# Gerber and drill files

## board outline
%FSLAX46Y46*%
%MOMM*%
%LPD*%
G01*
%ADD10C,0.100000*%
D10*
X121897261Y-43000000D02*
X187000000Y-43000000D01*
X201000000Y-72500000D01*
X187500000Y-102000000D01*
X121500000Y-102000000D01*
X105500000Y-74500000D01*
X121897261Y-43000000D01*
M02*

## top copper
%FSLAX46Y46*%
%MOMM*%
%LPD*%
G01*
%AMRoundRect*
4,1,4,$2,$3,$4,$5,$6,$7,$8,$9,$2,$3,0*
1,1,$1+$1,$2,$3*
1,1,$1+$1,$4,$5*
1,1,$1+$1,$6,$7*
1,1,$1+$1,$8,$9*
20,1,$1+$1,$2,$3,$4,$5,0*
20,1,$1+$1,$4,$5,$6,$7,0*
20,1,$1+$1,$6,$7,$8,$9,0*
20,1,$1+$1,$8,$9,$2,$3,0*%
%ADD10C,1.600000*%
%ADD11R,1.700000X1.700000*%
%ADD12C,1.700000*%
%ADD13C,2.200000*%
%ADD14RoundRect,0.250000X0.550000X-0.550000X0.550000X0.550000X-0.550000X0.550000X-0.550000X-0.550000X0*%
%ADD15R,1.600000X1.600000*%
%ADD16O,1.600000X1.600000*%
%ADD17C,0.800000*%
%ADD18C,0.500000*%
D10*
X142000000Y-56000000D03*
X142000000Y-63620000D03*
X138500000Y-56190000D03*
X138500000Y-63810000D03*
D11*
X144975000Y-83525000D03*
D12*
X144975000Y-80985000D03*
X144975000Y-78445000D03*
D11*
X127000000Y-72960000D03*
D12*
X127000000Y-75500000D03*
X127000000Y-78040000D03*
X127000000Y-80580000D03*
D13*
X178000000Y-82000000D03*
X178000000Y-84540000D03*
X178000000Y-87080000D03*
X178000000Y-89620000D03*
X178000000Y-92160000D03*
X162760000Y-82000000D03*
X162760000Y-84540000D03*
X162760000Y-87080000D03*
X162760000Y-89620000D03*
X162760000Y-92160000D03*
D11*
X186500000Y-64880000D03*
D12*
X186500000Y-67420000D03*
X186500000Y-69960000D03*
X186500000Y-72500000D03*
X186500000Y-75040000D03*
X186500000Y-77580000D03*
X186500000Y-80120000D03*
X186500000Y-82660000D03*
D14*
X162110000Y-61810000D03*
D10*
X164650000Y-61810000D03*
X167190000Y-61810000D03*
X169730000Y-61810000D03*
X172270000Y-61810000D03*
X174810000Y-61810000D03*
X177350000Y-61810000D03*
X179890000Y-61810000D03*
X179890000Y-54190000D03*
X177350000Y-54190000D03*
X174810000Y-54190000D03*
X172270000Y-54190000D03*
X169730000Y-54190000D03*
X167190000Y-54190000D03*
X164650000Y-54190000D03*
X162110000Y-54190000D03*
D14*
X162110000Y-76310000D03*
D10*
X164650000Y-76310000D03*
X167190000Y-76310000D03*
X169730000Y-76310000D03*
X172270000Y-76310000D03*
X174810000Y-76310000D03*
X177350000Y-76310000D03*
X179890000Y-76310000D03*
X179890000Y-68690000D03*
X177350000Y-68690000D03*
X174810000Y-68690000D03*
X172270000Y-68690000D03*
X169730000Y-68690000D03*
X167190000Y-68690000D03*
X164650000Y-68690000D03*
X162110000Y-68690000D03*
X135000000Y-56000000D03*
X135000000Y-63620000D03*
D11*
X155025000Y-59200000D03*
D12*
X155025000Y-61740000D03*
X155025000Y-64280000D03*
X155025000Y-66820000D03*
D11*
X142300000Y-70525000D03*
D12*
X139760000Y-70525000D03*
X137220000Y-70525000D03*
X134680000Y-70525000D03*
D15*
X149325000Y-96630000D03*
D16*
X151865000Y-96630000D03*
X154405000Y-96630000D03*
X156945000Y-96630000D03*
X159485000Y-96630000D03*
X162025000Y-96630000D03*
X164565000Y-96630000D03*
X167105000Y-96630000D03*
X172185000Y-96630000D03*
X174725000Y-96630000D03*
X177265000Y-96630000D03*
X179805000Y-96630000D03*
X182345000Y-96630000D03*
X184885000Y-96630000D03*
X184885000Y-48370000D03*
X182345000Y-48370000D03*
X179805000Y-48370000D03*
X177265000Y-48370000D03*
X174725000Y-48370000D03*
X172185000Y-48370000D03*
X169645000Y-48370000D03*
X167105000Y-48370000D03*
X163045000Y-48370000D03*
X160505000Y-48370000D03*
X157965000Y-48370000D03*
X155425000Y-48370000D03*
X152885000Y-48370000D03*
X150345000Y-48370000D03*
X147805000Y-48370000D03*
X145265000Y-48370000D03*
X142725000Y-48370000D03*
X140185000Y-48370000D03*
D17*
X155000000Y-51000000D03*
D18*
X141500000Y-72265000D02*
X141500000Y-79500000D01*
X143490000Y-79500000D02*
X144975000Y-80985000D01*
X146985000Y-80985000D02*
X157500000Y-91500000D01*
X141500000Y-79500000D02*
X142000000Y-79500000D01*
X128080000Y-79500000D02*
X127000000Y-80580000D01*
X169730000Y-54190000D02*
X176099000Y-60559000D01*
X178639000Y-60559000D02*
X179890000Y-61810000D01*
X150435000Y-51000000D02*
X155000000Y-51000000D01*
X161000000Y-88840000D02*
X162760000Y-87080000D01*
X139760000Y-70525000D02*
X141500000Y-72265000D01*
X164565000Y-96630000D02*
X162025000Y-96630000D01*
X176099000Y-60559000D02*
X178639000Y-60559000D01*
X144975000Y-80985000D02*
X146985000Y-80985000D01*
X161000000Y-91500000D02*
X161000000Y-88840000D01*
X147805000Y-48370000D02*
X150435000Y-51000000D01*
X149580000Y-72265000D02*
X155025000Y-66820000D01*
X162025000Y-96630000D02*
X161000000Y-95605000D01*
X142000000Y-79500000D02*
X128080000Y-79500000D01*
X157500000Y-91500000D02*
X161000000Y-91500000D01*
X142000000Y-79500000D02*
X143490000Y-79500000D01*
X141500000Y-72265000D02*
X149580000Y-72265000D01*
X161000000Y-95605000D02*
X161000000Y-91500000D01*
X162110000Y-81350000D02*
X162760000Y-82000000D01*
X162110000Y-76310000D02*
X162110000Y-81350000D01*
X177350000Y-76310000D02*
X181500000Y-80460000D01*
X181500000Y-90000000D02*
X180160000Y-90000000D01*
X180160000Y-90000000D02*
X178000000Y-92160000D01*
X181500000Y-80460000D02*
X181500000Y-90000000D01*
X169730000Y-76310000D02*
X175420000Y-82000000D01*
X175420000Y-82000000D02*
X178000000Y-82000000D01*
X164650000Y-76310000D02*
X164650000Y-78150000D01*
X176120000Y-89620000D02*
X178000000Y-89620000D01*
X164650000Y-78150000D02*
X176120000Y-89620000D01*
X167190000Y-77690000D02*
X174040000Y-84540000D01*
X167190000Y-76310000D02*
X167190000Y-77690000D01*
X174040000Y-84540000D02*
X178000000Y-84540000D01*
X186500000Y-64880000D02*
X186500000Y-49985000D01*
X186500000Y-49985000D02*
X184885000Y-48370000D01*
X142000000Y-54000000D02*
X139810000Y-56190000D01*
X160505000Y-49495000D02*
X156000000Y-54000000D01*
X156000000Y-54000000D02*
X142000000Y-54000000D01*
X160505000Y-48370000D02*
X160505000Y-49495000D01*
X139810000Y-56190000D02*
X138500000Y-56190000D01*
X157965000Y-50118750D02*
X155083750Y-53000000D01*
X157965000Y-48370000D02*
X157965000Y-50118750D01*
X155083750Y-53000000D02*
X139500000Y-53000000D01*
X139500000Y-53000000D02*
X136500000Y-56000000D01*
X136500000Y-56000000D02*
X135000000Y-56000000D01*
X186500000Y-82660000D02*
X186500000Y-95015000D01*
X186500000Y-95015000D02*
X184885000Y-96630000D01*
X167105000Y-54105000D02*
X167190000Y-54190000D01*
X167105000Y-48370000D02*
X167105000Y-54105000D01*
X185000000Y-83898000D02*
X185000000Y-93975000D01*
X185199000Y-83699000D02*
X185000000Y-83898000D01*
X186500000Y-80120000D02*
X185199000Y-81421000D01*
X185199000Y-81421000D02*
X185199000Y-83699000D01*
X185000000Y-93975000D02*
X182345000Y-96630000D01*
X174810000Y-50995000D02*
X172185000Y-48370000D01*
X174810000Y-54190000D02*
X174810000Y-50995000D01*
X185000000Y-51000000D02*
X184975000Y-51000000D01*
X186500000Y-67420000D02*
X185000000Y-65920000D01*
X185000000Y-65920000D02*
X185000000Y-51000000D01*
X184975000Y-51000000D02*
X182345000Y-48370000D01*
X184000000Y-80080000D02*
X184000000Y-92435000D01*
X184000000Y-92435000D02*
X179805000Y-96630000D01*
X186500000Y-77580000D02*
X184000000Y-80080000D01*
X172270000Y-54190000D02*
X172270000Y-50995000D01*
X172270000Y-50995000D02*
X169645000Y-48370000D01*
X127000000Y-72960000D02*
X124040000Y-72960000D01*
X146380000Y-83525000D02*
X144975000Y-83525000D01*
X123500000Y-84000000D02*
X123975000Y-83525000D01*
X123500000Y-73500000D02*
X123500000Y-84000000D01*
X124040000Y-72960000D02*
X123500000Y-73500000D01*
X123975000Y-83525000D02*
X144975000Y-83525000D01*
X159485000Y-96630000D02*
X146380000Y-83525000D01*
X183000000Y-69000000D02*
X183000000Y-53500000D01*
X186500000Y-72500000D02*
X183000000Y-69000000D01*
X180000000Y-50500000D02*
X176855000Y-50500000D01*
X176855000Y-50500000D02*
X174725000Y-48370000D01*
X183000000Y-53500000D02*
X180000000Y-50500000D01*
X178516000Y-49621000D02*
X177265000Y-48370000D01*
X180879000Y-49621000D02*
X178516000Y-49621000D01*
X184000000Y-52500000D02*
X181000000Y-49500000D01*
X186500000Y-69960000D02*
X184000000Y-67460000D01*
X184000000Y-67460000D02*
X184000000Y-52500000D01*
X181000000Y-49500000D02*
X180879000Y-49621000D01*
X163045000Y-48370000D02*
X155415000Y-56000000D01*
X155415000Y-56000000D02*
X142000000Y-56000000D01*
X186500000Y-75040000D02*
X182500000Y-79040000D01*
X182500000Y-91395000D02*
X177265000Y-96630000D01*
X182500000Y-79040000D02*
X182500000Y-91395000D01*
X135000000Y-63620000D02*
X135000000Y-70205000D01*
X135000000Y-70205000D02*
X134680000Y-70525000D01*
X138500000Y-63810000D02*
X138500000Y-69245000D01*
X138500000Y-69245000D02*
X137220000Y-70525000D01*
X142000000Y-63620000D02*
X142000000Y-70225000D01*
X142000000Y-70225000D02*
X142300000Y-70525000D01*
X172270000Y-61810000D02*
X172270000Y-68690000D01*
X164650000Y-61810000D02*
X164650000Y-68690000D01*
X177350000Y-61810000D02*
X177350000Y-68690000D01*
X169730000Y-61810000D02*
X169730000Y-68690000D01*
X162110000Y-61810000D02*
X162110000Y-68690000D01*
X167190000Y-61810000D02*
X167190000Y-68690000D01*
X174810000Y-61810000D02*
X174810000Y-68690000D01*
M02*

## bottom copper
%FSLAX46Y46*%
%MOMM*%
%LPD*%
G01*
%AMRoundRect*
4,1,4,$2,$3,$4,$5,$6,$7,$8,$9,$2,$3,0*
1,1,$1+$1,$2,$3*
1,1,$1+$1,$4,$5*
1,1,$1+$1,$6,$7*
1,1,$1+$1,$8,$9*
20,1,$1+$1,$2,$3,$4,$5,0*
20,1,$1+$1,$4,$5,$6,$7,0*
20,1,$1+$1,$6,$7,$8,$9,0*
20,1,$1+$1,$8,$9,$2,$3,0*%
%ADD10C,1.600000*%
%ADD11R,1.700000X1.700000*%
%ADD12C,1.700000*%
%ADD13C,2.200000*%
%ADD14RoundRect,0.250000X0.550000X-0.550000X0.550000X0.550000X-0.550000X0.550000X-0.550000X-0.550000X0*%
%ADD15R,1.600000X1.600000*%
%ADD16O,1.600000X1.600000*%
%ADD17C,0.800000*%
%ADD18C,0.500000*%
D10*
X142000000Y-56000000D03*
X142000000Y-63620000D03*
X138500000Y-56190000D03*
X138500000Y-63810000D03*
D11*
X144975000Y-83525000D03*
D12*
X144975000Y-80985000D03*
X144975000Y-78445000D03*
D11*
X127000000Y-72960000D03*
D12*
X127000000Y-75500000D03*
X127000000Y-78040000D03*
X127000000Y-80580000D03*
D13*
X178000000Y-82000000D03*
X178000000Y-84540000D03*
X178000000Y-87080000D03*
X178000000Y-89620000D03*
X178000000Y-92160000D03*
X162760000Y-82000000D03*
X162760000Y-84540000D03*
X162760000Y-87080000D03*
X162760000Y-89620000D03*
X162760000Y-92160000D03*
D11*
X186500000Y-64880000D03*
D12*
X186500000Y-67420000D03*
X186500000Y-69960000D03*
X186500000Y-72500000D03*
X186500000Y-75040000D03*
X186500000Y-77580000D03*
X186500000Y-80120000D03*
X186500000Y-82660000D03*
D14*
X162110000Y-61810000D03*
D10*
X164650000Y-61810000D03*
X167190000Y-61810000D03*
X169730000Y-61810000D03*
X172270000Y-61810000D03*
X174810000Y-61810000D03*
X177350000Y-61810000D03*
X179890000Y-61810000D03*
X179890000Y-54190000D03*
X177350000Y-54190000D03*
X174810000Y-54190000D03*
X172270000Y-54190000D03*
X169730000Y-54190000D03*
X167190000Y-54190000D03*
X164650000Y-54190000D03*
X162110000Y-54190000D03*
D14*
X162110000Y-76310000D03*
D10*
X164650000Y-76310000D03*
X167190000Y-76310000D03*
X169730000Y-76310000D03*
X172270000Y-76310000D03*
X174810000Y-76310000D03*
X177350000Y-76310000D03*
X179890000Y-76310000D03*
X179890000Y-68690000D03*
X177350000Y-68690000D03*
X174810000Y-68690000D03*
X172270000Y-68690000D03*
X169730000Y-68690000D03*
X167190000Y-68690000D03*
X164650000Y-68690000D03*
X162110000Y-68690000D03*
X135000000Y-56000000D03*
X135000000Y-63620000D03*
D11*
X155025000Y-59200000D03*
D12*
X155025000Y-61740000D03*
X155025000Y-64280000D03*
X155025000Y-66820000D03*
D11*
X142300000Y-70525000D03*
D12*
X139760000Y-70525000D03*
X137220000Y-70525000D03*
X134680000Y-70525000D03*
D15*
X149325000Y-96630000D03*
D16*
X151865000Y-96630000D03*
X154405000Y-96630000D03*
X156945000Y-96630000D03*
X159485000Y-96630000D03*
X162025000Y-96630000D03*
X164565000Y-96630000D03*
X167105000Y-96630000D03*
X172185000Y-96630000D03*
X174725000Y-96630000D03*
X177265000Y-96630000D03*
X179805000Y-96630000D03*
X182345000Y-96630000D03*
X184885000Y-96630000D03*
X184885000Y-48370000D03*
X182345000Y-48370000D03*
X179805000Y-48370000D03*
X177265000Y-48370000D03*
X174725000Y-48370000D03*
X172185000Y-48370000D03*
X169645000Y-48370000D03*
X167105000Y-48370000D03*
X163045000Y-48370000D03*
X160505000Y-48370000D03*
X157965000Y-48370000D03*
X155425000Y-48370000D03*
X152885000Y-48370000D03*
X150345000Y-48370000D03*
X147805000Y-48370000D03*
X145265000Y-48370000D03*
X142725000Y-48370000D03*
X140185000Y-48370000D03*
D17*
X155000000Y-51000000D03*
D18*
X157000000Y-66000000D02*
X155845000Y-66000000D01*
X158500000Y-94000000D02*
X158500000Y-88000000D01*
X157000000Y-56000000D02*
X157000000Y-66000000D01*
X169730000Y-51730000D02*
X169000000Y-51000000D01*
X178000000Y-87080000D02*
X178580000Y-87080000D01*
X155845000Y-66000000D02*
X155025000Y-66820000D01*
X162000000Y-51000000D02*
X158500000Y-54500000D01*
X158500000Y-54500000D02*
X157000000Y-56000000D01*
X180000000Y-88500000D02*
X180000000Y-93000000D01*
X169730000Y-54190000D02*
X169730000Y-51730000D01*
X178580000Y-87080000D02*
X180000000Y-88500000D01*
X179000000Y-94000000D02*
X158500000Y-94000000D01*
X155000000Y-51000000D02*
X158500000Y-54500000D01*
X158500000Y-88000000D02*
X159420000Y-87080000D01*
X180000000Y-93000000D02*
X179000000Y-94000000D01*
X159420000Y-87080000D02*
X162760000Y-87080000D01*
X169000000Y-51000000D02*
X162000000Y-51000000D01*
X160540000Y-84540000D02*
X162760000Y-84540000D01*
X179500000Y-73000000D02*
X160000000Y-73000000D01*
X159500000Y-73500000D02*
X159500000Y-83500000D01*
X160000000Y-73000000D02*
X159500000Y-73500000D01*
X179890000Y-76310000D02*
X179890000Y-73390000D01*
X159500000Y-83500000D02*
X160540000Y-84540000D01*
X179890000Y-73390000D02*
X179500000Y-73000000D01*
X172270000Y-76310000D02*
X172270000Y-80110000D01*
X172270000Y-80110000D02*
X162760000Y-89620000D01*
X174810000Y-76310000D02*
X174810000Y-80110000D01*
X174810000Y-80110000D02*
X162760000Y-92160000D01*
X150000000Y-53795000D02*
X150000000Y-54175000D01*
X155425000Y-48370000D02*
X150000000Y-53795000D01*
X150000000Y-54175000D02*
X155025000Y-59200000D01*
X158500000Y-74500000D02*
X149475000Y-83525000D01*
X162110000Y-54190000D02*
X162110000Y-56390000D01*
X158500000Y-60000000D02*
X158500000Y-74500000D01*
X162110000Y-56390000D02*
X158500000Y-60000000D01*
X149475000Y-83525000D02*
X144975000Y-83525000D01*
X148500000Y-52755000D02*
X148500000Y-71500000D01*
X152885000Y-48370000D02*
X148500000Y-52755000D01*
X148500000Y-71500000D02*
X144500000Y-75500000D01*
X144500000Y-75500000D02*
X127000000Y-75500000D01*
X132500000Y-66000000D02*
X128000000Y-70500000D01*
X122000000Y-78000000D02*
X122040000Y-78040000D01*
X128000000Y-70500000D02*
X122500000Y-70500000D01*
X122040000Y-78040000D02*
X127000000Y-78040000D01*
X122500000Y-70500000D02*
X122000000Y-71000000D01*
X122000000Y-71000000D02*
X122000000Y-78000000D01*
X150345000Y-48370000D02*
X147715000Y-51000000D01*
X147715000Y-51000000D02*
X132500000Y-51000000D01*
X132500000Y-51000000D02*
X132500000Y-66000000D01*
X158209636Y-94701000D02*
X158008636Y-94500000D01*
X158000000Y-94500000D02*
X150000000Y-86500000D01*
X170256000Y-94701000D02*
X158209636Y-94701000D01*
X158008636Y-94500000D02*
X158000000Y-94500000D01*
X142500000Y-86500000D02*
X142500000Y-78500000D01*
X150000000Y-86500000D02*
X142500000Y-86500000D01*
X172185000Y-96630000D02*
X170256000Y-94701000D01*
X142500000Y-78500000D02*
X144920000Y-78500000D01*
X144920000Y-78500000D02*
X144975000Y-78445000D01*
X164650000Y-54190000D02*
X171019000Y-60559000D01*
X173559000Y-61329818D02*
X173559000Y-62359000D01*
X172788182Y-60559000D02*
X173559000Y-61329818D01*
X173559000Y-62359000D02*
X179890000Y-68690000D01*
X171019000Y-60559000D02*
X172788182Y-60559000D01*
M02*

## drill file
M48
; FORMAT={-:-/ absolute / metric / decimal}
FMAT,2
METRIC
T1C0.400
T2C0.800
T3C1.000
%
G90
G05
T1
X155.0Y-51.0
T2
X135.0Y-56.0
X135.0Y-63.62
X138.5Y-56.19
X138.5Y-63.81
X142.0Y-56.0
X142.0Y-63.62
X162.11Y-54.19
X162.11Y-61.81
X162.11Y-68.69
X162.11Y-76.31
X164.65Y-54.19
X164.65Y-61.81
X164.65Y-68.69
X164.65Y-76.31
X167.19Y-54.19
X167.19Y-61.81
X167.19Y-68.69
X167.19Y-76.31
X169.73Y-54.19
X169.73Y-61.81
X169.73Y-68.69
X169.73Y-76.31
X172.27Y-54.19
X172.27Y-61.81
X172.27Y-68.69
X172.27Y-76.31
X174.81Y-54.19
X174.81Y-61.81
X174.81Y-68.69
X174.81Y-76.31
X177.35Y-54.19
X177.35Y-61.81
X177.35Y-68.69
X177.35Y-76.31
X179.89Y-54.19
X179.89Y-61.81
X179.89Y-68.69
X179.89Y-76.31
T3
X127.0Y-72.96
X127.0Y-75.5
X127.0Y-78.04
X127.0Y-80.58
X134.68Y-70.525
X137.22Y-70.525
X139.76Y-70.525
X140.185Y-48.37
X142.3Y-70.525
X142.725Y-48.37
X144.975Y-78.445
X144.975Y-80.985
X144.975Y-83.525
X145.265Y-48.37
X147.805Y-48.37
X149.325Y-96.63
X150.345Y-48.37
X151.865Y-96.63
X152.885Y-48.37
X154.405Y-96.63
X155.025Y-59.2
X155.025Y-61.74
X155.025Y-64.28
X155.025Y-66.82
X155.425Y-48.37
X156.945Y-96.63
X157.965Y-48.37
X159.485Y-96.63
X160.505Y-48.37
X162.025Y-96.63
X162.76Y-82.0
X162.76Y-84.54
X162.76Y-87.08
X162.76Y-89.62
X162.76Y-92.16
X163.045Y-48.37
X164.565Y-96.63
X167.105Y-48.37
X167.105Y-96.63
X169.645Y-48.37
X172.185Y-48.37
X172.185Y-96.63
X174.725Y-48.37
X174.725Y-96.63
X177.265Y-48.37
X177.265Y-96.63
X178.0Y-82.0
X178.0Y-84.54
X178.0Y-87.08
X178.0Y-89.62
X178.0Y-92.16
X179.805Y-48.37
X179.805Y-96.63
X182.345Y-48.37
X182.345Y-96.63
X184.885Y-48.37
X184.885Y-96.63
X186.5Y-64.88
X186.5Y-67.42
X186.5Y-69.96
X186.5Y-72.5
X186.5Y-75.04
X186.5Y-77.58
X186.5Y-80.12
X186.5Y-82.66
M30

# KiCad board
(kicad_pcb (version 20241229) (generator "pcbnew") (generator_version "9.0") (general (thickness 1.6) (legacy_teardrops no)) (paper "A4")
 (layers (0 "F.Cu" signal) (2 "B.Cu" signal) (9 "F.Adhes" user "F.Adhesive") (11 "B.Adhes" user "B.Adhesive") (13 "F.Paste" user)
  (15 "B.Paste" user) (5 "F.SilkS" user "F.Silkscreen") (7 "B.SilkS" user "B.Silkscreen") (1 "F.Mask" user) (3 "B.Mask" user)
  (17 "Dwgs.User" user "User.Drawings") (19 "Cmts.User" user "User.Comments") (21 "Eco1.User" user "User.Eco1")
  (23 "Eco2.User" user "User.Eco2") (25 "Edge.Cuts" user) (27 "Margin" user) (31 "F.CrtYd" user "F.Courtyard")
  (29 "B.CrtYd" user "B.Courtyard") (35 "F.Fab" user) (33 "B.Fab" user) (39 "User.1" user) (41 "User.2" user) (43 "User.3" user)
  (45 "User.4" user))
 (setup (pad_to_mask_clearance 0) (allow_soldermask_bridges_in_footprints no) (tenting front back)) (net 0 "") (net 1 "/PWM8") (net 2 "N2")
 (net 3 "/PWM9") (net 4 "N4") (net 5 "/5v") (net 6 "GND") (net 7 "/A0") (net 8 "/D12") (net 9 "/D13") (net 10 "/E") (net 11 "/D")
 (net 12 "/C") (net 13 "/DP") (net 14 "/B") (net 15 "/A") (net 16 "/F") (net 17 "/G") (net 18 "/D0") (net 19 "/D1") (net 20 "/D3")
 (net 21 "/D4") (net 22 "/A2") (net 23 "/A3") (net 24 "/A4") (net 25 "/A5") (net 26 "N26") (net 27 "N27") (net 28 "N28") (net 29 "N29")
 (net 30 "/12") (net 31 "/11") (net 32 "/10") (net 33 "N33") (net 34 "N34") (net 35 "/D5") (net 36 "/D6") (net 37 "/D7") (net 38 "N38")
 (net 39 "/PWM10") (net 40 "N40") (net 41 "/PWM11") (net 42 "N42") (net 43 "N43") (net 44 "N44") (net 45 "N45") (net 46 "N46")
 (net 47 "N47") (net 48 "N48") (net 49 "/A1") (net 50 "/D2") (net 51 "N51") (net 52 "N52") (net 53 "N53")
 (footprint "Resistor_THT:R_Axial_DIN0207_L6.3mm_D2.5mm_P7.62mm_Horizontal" (layer "F.Cu") (at 142 56 -90)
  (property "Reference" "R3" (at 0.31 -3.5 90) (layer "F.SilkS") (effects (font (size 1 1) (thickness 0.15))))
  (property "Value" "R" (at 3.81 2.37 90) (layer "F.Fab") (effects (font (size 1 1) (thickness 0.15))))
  (pad "1" thru_hole circle (at 0 0 270) (size 1.6 1.6) (drill 0.8) (layers "*.Cu" "*.Mask") (remove_unused_layers no) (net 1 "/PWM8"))
  (pad "2" thru_hole circle (at 7.62 0 270) (size 1.6 1.6) (drill 0.8) (layers "*.Cu" "*.Mask") (remove_unused_layers no) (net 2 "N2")))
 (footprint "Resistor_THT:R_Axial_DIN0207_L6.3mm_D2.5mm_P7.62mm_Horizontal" (layer "F.Cu") (at 138.5 56.19 -90)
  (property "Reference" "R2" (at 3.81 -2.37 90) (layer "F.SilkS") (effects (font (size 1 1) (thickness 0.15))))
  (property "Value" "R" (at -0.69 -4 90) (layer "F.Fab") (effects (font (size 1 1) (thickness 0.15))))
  (pad "1" thru_hole circle (at 0 0 270) (size 1.6 1.6) (drill 0.8) (layers "*.Cu" "*.Mask") (remove_unused_layers no) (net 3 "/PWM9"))
  (pad "2" thru_hole circle (at 7.62 0 270) (size 1.6 1.6) (drill 0.8) (layers "*.Cu" "*.Mask") (remove_unused_layers no) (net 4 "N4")))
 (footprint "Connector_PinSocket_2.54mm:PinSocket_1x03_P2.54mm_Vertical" (layer "F.Cu") (at 144.975 83.525 180)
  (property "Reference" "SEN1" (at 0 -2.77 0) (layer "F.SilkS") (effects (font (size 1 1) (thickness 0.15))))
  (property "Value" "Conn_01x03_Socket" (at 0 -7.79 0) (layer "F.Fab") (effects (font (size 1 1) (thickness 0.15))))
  (pad "1" thru_hole rect (at 0 0 180) (size 1.7 1.7) (drill 1) (layers "*.Cu" "*.Mask") (remove_unused_layers no) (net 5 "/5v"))
  (pad "2" thru_hole circle (at 0 2.54 180) (size 1.7 1.7) (drill 1) (layers "*.Cu" "*.Mask") (remove_unused_layers no) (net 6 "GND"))
  (pad "3" thru_hole circle (at 0 5.08 180) (size 1.7 1.7) (drill 1) (layers "*.Cu" "*.Mask") (remove_unused_layers no) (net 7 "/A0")))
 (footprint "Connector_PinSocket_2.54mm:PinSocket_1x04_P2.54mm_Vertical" (layer "F.Cu") (at 127 72.96)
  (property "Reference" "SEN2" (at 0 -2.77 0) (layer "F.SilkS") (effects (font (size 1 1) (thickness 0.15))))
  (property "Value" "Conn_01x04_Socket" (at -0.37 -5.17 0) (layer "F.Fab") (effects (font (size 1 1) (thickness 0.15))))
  (pad "1" thru_hole rect (at 0 0) (size 1.7 1.7) (drill 1) (layers "*.Cu" "*.Mask") (remove_unused_layers no) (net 5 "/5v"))
  (pad "2" thru_hole circle (at 0 2.54) (size 1.7 1.7) (drill 1) (layers "*.Cu" "*.Mask") (remove_unused_layers no) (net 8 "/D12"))
  (pad "3" thru_hole circle (at 0 5.08) (size 1.7 1.7) (drill 1) (layers "*.Cu" "*.Mask") (remove_unused_layers no) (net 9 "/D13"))
  (pad "4" thru_hole circle (at 0 7.62) (size 1.7 1.7) (drill 1) (layers "*.Cu" "*.Mask") (remove_unused_layers no) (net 6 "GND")))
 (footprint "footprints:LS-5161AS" (layer "F.Cu") (at 178 82 -90)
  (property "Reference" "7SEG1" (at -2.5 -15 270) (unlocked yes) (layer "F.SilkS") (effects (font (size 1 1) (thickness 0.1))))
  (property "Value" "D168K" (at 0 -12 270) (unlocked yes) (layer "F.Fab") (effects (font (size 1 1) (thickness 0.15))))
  (pad "1" thru_hole circle (at 0 0 270) (size 2.2 2.2) (drill 1) (layers "*.Cu" "*.Mask") (remove_unused_layers no) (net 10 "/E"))
  (pad "2" thru_hole circle (at 2.54 0 270) (size 2.2 2.2) (drill 1) (layers "*.Cu" "*.Mask") (remove_unused_layers no) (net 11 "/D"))
  (pad "3" thru_hole circle (at 5.08 0 270) (size 2.2 2.2) (drill 1) (layers "*.Cu" "*.Mask") (remove_unused_layers no) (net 6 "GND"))
  (pad "4" thru_hole circle (at 7.62 0 270) (size 2.2 2.2) (drill 1) (layers "*.Cu" "*.Mask") (remove_unused_layers no) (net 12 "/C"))
  (pad "5" thru_hole circle (at 10.16 0 270) (size 2.2 2.2) (drill 1) (layers "*.Cu" "*.Mask") (remove_unused_layers no) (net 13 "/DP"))
  (pad "6" thru_hole circle (at 0 15.24 270) (size 2.2 2.2) (drill 1) (layers "*.Cu" "*.Mask") (remove_unused_layers no) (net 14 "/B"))
  (pad "7" thru_hole circle (at 2.54 15.24 270) (size 2.2 2.2) (drill 1) (layers "*.Cu" "*.Mask") (remove_unused_layers no) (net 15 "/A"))
  (pad "8" thru_hole circle (at 5.08 15.24 270) (size 2.2 2.2) (drill 1) (layers "*.Cu" "*.Mask") (remove_unused_layers no) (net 6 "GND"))
  (pad "9" thru_hole circle (at 7.62 15.24 270) (size 2.2 2.2) (drill 1) (layers "*.Cu" "*.Mask") (remove_unused_layers no) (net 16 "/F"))
  (pad "10" thru_hole circle (at 10.16 15.24 270) (size 2.2 2.2) (drill 1) (layers "*.Cu" "*.Mask") (remove_unused_layers no) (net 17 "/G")))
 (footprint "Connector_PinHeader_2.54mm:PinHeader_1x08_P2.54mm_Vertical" (layer "F.Cu") (at 186.5 64.88)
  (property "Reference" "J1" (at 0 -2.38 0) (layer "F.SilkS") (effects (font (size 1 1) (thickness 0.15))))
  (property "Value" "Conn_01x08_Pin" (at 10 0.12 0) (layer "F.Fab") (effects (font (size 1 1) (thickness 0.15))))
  (pad "1" thru_hole rect (at 0 0) (size 1.7 1.7) (drill 1) (layers "*.Cu" "*.Mask") (remove_unused_layers no) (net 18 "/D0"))
  (pad "2" thru_hole circle (at 0 2.54) (size 1.7 1.7) (drill 1) (layers "*.Cu" "*.Mask") (remove_unused_layers no) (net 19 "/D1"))
  (pad "3" thru_hole circle (at 0 5.08) (size 1.7 1.7) (drill 1) (layers "*.Cu" "*.Mask") (remove_unused_layers no) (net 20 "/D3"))
  (pad "4" thru_hole circle (at 0 7.62) (size 1.7 1.7) (drill 1) (layers "*.Cu" "*.Mask") (remove_unused_layers no) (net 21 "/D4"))
  (pad "5" thru_hole circle (at 0 10.16) (size 1.7 1.7) (drill 1) (layers "*.Cu" "*.Mask") (remove_unused_layers no) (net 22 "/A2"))
  (pad "6" thru_hole circle (at 0 12.7) (size 1.7 1.7) (drill 1) (layers "*.Cu" "*.Mask") (remove_unused_layers no) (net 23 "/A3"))
  (pad "7" thru_hole circle (at 0 15.24) (size 1.7 1.7) (drill 1) (layers "*.Cu" "*.Mask") (remove_unused_layers no) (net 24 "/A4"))
  (pad "8" thru_hole circle (at 0 17.78) (size 1.7 1.7) (drill 1) (layers "*.Cu" "*.Mask") (remove_unused_layers no) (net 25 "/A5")))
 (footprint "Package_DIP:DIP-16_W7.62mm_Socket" (layer "F.Cu") (at 162.11 61.81 90)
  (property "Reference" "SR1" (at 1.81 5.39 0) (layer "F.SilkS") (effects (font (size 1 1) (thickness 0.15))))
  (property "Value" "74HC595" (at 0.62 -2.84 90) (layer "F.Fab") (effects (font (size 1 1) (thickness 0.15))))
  (pad "1" thru_hole roundrect (at 0 0 90) (size 1.6 1.6) (drill 0.8) (layers "*.Cu" "*.Mask") (remove_unused_layers no)
   (roundrect_rratio 0.15625) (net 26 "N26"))
  (pad "2" thru_hole circle (at 0 2.54 90) (size 1.6 1.6) (drill 0.8) (layers "*.Cu" "*.Mask") (remove_unused_layers no) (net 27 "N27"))
  (pad "3" thru_hole circle (at 0 5.08 90) (size 1.6 1.6) (drill 0.8) (layers "*.Cu" "*.Mask") (remove_unused_layers no) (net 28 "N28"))
  (pad "4" thru_hole circle (at 0 7.62 90) (size 1.6 1.6) (drill 0.8) (layers "*.Cu" "*.Mask") (remove_unused_layers no) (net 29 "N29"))
  (pad "5" thru_hole circle (at 0 10.16 90) (size 1.6 1.6) (drill 0.8) (layers "*.Cu" "*.Mask") (remove_unused_layers no) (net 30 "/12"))
  (pad "6" thru_hole circle (at 0 12.7 90) (size 1.6 1.6) (drill 0.8) (layers "*.Cu" "*.Mask") (remove_unused_layers no) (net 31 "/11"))
  (pad "7" thru_hole circle (at 0 15.24 90) (size 1.6 1.6) (drill 0.8) (layers "*.Cu" "*.Mask") (remove_unused_layers no) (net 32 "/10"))
  (pad "8" thru_hole circle (at 0 17.78 90) (size 1.6 1.6) (drill 0.8) (layers "*.Cu" "*.Mask") (remove_unused_layers no) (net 6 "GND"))
  (pad "9" thru_hole circle (at 7.62 17.78 90) (size 1.6 1.6) (drill 0.8) (layers "*.Cu" "*.Mask") (remove_unused_layers no) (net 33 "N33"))
  (pad "10" thru_hole circle (at 7.62 15.24 90) (size 1.6 1.6) (drill 0.8) (layers "*.Cu" "*.Mask") (remove_unused_layers no) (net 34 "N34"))
  (pad "11" thru_hole circle (at 7.62 12.7 90) (size 1.6 1.6) (drill 0.8) (layers "*.Cu" "*.Mask") (remove_unused_layers no) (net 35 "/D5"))
  (pad "12" thru_hole circle (at 7.62 10.16 90) (size 1.6 1.6) (drill 0.8) (layers "*.Cu" "*.Mask") (remove_unused_layers no) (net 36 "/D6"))
  (pad "13" thru_hole circle (at 7.62 7.62 90) (size 1.6 1.6) (drill 0.8) (layers "*.Cu" "*.Mask") (remove_unused_layers no) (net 6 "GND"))
  (pad "14" thru_hole circle (at 7.62 5.08 90) (size 1.6 1.6) (drill 0.8) (layers "*.Cu" "*.Mask") (remove_unused_layers no) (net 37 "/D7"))
  (pad "15" thru_hole circle (at 7.62 2.54 90) (size 1.6 1.6) (drill 0.8) (layers "*.Cu" "*.Mask") (remove_unused_layers no) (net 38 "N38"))
  (pad "16" thru_hole circle (at 7.62 0 90) (size 1.6 1.6) (drill 0.8) (layers "*.Cu" "*.Mask") (remove_unused_layers no) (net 5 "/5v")))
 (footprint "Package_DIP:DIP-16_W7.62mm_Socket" (layer "F.Cu") (at 162.11 76.31 90)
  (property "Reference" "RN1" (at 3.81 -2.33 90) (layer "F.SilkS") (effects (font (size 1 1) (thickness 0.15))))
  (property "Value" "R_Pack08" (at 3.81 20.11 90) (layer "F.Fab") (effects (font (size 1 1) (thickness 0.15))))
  (pad "1" thru_hole roundrect (at 0 0 90) (size 1.6 1.6) (drill 0.8) (layers "*.Cu" "*.Mask") (remove_unused_layers no)
   (roundrect_rratio 0.15625) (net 14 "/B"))
  (pad "2" thru_hole circle (at 0 2.54 90) (size 1.6 1.6) (drill 0.8) (layers "*.Cu" "*.Mask") (remove_unused_layers no) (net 12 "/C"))
  (pad "3" thru_hole circle (at 0 5.08 90) (size 1.6 1.6) (drill 0.8) (layers "*.Cu" "*.Mask") (remove_unused_layers no) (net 11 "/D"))
  (pad "4" thru_hole circle (at 0 7.62 90) (size 1.6 1.6) (drill 0.8) (layers "*.Cu" "*.Mask") (remove_unused_layers no) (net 10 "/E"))
  (pad "5" thru_hole circle (at 0 10.16 90) (size 1.6 1.6) (drill 0.8) (layers "*.Cu" "*.Mask") (remove_unused_layers no) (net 16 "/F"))
  (pad "6" thru_hole circle (at 0 12.7 90) (size 1.6 1.6) (drill 0.8) (layers "*.Cu" "*.Mask") (remove_unused_layers no) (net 17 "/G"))
  (pad "7" thru_hole circle (at 0 15.24 90) (size 1.6 1.6) (drill 0.8) (layers "*.Cu" "*.Mask") (remove_unused_layers no) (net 13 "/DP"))
  (pad "8" thru_hole circle (at 0 17.78 90) (size 1.6 1.6) (drill 0.8) (layers "*.Cu" "*.Mask") (remove_unused_layers no) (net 15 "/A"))
  (pad "9" thru_hole circle (at 7.62 17.78 90) (size 1.6 1.6) (drill 0.8) (layers "*.Cu" "*.Mask") (remove_unused_layers no) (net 38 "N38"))
  (pad "10" thru_hole circle (at 7.62 15.24 90) (size 1.6 1.6) (drill 0.8) (layers "*.Cu" "*.Mask") (remove_unused_layers no) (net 32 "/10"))
  (pad "11" thru_hole circle (at 7.62 12.7 90) (size 1.6 1.6) (drill 0.8) (layers "*.Cu" "*.Mask") (remove_unused_layers no) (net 31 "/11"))
  (pad "12" thru_hole circle (at 7.62 10.16 90) (size 1.6 1.6) (drill 0.8) (layers "*.Cu" "*.Mask") (remove_unused_layers no) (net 30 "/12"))
  (pad "13" thru_hole circle (at 7.62 7.62 90) (size 1.6 1.6) (drill 0.8) (layers "*.Cu" "*.Mask") (remove_unused_layers no) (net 29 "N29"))
  (pad "14" thru_hole circle (at 7.62 5.08 90) (size 1.6 1.6) (drill 0.8) (layers "*.Cu" "*.Mask") (remove_unused_layers no) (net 28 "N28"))
  (pad "15" thru_hole circle (at 7.62 2.54 90) (size 1.6 1.6) (drill 0.8) (layers "*.Cu" "*.Mask") (remove_unused_layers no) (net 27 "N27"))
  (pad "16" thru_hole circle (at 7.62 0 90) (size 1.6 1.6) (drill 0.8) (layers "*.Cu" "*.Mask") (remove_unused_layers no) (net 26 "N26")))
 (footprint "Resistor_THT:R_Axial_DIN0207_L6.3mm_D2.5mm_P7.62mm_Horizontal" (layer "F.Cu") (at 135 56 -90)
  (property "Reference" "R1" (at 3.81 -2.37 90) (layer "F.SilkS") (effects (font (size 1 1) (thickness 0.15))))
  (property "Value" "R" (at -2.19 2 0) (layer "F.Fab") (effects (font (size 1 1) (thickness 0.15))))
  (pad "1" thru_hole circle (at 0 0 270) (size 1.6 1.6) (drill 0.8) (layers "*.Cu" "*.Mask") (remove_unused_layers no) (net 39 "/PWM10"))
  (pad "2" thru_hole circle (at 7.62 0 270) (size 1.6 1.6) (drill 0.8) (layers "*.Cu" "*.Mask") (remove_unused_layers no) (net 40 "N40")))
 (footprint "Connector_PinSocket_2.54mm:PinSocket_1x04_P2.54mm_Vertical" (layer "F.Cu") (at 155.025 59.2)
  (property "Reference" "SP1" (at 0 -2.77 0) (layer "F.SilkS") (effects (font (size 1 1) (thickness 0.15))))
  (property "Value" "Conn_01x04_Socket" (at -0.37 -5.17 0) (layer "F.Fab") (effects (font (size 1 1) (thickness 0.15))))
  (pad "1" thru_hole rect (at 0 0) (size 1.7 1.7) (drill 1) (layers "*.Cu" "*.Mask") (remove_unused_layers no) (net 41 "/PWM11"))
  (pad "2" thru_hole circle (at 0 2.54) (size 1.7 1.7) (drill 1) (layers "*.Cu" "*.Mask") (remove_unused_layers no) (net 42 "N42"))
  (pad "3" thru_hole circle (at 0 5.08) (size 1.7 1.7) (drill 1) (layers "*.Cu" "*.Mask") (remove_unused_layers no) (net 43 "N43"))
  (pad "4" thru_hole circle (at 0 7.62) (size 1.7 1.7) (drill 1) (layers "*.Cu" "*.Mask") (remove_unused_layers no) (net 6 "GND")))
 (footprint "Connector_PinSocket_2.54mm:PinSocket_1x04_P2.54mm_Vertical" (layer "F.Cu") (at 142.3 70.525 -90)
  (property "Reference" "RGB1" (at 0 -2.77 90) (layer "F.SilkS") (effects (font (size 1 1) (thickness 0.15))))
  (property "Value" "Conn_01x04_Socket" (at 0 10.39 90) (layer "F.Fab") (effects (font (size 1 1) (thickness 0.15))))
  (pad "1" thru_hole rect (at 0 0 270) (size 1.7 1.7) (drill 1) (layers "*.Cu" "*.Mask") (remove_unused_layers no) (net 2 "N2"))
  (pad "2" thru_hole circle (at 0 2.54 270) (size 1.7 1.7) (drill 1) (layers "*.Cu" "*.Mask") (remove_unused_layers no) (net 6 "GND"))
  (pad "3" thru_hole circle (at 0 5.08 270) (size 1.7 1.7) (drill 1) (layers "*.Cu" "*.Mask") (remove_unused_layers no) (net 4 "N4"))
  (pad "4" thru_hole circle (at 0 7.62 270) (size 1.7 1.7) (drill 1) (layers "*.Cu" "*.Mask") (remove_unused_layers no) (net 40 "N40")))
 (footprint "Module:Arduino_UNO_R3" (layer "B.Cu") (at 149.325 96.63)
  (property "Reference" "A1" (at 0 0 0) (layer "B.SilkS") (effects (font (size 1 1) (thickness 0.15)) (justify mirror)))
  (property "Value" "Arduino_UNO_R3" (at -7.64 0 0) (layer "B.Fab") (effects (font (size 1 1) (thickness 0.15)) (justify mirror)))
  (pad "1" thru_hole rect (at 0 0 270) (size 1.6 1.6) (drill 1) (layers "*.Cu" "*.Mask") (remove_unused_layers no) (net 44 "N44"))
  (pad "2" thru_hole oval (at 2.54 0 270) (size 1.6 1.6) (drill 1) (layers "*.Cu" "*.Mask") (remove_unused_layers no) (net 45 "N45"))
  (pad "3" thru_hole oval (at 5.08 0 270) (size 1.6 1.6) (drill 1) (layers "*.Cu" "*.Mask") (remove_unused_layers no) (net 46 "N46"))
  (pad "4" thru_hole oval (at 7.62 0 270) (size 1.6 1.6) (drill 1) (layers "*.Cu" "*.Mask") (remove_unused_layers no) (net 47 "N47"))
  (pad "5" thru_hole oval (at 10.16 0 270) (size 1.6 1.6) (drill 1) (layers "*.Cu" "*.Mask") (remove_unused_layers no) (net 5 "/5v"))
  (pad "6" thru_hole oval (at 12.7 0 270) (size 1.6 1.6) (drill 1) (layers "*.Cu" "*.Mask") (remove_unused_layers no) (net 6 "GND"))
  (pad "7" thru_hole oval (at 15.24 0 270) (size 1.6 1.6) (drill 1) (layers "*.Cu" "*.Mask") (remove_unused_layers no) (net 6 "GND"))
  (pad "8" thru_hole oval (at 17.78 0 270) (size 1.6 1.6) (drill 1) (layers "*.Cu" "*.Mask") (remove_unused_layers no) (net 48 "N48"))
  (pad "9" thru_hole oval (at 22.86 0 270) (size 1.6 1.6) (drill 1) (layers "*.Cu" "*.Mask") (remove_unused_layers no) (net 7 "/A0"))
  (pad "10" thru_hole oval (at 25.4 0 270) (size 1.6 1.6) (drill 1) (layers "*.Cu" "*.Mask") (remove_unused_layers no) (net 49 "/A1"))
  (pad "11" thru_hole oval (at 27.94 0 270) (size 1.6 1.6) (drill 1) (layers "*.Cu" "*.Mask") (remove_unused_layers no) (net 22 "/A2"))
  (pad "12" thru_hole oval (at 30.48 0 270) (size 1.6 1.6) (drill 1) (layers "*.Cu" "*.Mask") (remove_unused_layers no) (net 23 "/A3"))
  (pad "13" thru_hole oval (at 33.02 0 270) (size 1.6 1.6) (drill 1) (layers "*.Cu" "*.Mask") (remove_unused_layers no) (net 24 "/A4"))
  (pad "14" thru_hole oval (at 35.56 0 270) (size 1.6 1.6) (drill 1) (layers "*.Cu" "*.Mask") (remove_unused_layers no) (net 25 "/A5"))
  (pad "15" thru_hole oval (at 35.56 -48.26 270) (size 1.6 1.6) (drill 1) (layers "*.Cu" "*.Mask") (remove_unused_layers no) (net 18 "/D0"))
  (pad "16" thru_hole oval (at 33.02 -48.26 270) (size 1.6 1.6) (drill 1) (layers "*.Cu" "*.Mask") (remove_unused_layers no) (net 19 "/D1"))
  (pad "17" thru_hole oval (at 30.48 -48.26 270) (size 1.6 1.6) (drill 1) (layers "*.Cu" "*.Mask") (remove_unused_layers no) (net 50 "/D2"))
  (pad "18" thru_hole oval (at 27.94 -48.26 270) (size 1.6 1.6) (drill 1) (layers "*.Cu" "*.Mask") (remove_unused_layers no) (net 20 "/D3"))
  (pad "19" thru_hole oval (at 25.4 -48.26 270) (size 1.6 1.6) (drill 1) (layers "*.Cu" "*.Mask") (remove_unused_layers no) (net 21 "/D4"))
  (pad "20" thru_hole oval (at 22.86 -48.26 270) (size 1.6 1.6) (drill 1) (layers "*.Cu" "*.Mask") (remove_unused_layers no) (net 35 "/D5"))
  (pad "21" thru_hole oval (at 20.32 -48.26 270) (size 1.6 1.6) (drill 1) (layers "*.Cu" "*.Mask") (remove_unused_layers no) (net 36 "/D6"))
  (pad "22" thru_hole oval (at 17.78 -48.26 270) (size 1.6 1.6) (drill 1) (layers "*.Cu" "*.Mask") (remove_unused_layers no) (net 37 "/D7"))
  (pad "23" thru_hole oval (at 13.72 -48.26 270) (size 1.6 1.6) (drill 1) (layers "*.Cu" "*.Mask") (remove_unused_layers no) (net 1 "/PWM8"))
  (pad "24" thru_hole oval (at 11.18 -48.26 270) (size 1.6 1.6) (drill 1) (layers "*.Cu" "*.Mask") (remove_unused_layers no) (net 3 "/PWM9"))
  (pad "25" thru_hole oval (at 8.64 -48.26 270) (size 1.6 1.6) (drill 1) (layers "*.Cu" "*.Mask") (remove_unused_layers no)
   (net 39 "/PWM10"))
  (pad "26" thru_hole oval (at 6.1 -48.26 270) (size 1.6 1.6) (drill 1) (layers "*.Cu" "*.Mask") (remove_unused_layers no) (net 41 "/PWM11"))
  (pad "27" thru_hole oval (at 3.56 -48.26 270) (size 1.6 1.6) (drill 1) (layers "*.Cu" "*.Mask") (remove_unused_layers no) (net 8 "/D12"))
  (pad "28" thru_hole oval (at 1.02 -48.26 270) (size 1.6 1.6) (drill 1) (layers "*.Cu" "*.Mask") (remove_unused_layers no) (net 9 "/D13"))
  (pad "29" thru_hole oval (at -1.52 -48.26 270) (size 1.6 1.6) (drill 1) (layers "*.Cu" "*.Mask") (remove_unused_layers no) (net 6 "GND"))
  (pad "30" thru_hole oval (at -4.06 -48.26 270) (size 1.6 1.6) (drill 1) (layers "*.Cu" "*.Mask") (remove_unused_layers no) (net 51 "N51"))
  (pad "31" thru_hole oval (at -6.6 -48.26 270) (size 1.6 1.6) (drill 1) (layers "*.Cu" "*.Mask") (remove_unused_layers no) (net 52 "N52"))
  (pad "32" thru_hole oval (at -9.14 -48.26 270) (size 1.6 1.6) (drill 1) (layers "*.Cu" "*.Mask") (remove_unused_layers no) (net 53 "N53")))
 (gr_poly
  (pts (xy 121.897261 43) (xy 187 43) (xy 201 72.5) (xy 187.5 102) (xy 121.5 102) (xy 105.5 74.5)) (stroke (width 0.1) (type solid))
  (fill no) (layer "Edge.Cuts"))
 (segment (start 141.5 72.265) (end 141.5 79.5) (width 0.5) (layer "F.Cu") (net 6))
 (segment (start 143.49 79.5) (end 144.975 80.985) (width 0.5) (layer "F.Cu") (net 6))
 (segment (start 146.985 80.985) (end 157.5 91.5) (width 0.5) (layer "F.Cu") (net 6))
 (segment (start 141.5 79.5) (end 142 79.5) (width 0.5) (layer "F.Cu") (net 6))
 (segment (start 128.08 79.5) (end 127 80.58) (width 0.5) (layer "F.Cu") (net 6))
 (segment (start 169.73 54.19) (end 176.099 60.559) (width 0.5) (layer "F.Cu") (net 6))
 (segment (start 178.639 60.559) (end 179.89 61.81) (width 0.5) (layer "F.Cu") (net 6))
 (segment (start 150.435 51) (end 155 51) (width 0.5) (layer "F.Cu") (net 6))
 (segment (start 161 88.84) (end 162.76 87.08) (width 0.5) (layer "F.Cu") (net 6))
 (segment (start 139.76 70.525) (end 141.5 72.265) (width 0.5) (layer "F.Cu") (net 6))
 (segment (start 164.565 96.63) (end 162.025 96.63) (width 0.5) (layer "F.Cu") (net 6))
 (segment (start 176.099 60.559) (end 178.639 60.559) (width 0.5) (layer "F.Cu") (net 6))
 (segment (start 144.975 80.985) (end 146.985 80.985) (width 0.5) (layer "F.Cu") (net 6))
 (segment (start 161 91.5) (end 161 88.84) (width 0.5) (layer "F.Cu") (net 6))
 (segment (start 147.805 48.37) (end 150.435 51) (width 0.5) (layer "F.Cu") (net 6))
 (segment (start 149.58 72.265) (end 155.025 66.82) (width 0.5) (layer "F.Cu") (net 6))
 (segment (start 162.025 96.63) (end 161 95.605) (width 0.5) (layer "F.Cu") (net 6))
 (segment (start 142 79.5) (end 128.08 79.5) (width 0.5) (layer "F.Cu") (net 6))
 (segment (start 157.5 91.5) (end 161 91.5) (width 0.5) (layer "F.Cu") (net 6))
 (segment (start 142 79.5) (end 143.49 79.5) (width 0.5) (layer "F.Cu") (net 6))
 (segment (start 141.5 72.265) (end 149.58 72.265) (width 0.5) (layer "F.Cu") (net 6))
 (segment (start 161 95.605) (end 161 91.5) (width 0.5) (layer "F.Cu") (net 6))
 (via (at 155 51) (size 0.8) (drill 0.4) (layers "F.Cu" "B.Cu") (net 6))
 (segment (start 157 66) (end 155.845 66) (width 0.5) (layer "B.Cu") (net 6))
 (segment (start 158.5 94) (end 158.5 88) (width 0.5) (layer "B.Cu") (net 6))
 (segment (start 157 56) (end 157 66) (width 0.5) (layer "B.Cu") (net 6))
 (segment (start 169.73 51.73) (end 169 51) (width 0.5) (layer "B.Cu") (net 6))
 (segment (start 178 87.08) (end 178.58 87.08) (width 0.5) (layer "B.Cu") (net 6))
 (segment (start 155.845 66) (end 155.025 66.82) (width 0.5) (layer "B.Cu") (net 6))
 (segment (start 162 51) (end 158.5 54.5) (width 0.5) (layer "B.Cu") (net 6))
 (segment (start 158.5 54.5) (end 157 56) (width 0.5) (layer "B.Cu") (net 6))
 (segment (start 180 88.5) (end 180 93) (width 0.5) (layer "B.Cu") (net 6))
 (segment (start 169.73 54.19) (end 169.73 51.73) (width 0.5) (layer "B.Cu") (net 6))
 (segment (start 178.58 87.08) (end 180 88.5) (width 0.5) (layer "B.Cu") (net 6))
 (segment (start 179 94) (end 158.5 94) (width 0.5) (layer "B.Cu") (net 6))
 (segment (start 155 51) (end 158.5 54.5) (width 0.5) (layer "B.Cu") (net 6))
 (segment (start 158.5 88) (end 159.42 87.08) (width 0.5) (layer "B.Cu") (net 6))
 (segment (start 180 93) (end 179 94) (width 0.5) (layer "B.Cu") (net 6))
 (segment (start 159.42 87.08) (end 162.76 87.08) (width 0.5) (layer "B.Cu") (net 6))
 (segment (start 169 51) (end 162 51) (width 0.5) (layer "B.Cu") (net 6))
 (segment (start 160.54 84.54) (end 162.76 84.54) (width 0.5) (layer "B.Cu") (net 15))
 (segment (start 179.5 73) (end 160 73) (width 0.5) (layer "B.Cu") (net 15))
 (segment (start 159.5 73.5) (end 159.5 83.5) (width 0.5) (layer "B.Cu") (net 15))
 (segment (start 160 73) (end 159.5 73.5) (width 0.5) (layer "B.Cu") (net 15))
 (segment (start 179.89 76.31) (end 179.89 73.39) (width 0.5) (layer "B.Cu") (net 15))
 (segment (start 159.5 83.5) (end 160.54 84.54) (width 0.5) (layer "B.Cu") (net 15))
 (segment (start 179.89 73.39) (end 179.5 73) (width 0.5) (layer "B.Cu") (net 15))
 (segment (start 162.11 81.35) (end 162.76 82) (width 0.5) (layer "F.Cu") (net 14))
 (segment (start 162.11 76.31) (end 162.11 81.35) (width 0.5) (layer "F.Cu") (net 14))
 (segment (start 177.35 76.31) (end 181.5 80.46) (width 0.5) (layer "F.Cu") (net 13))
 (segment (start 181.5 90) (end 180.16 90) (width 0.5) (layer "F.Cu") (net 13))
 (segment (start 180.16 90) (end 178 92.16) (width 0.5) (layer "F.Cu") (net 13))
 (segment (start 181.5 80.46) (end 181.5 90) (width 0.5) (layer "F.Cu") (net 13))
 (segment (start 169.73 76.31) (end 175.42 82) (width 0.5) (layer "F.Cu") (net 10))
 (segment (start 175.42 82) (end 178 82) (width 0.5) (layer "F.Cu") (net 10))
 (segment (start 172.27 76.31) (end 172.27 80.11) (width 0.5) (layer "B.Cu") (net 16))
 (segment (start 172.27 80.11) (end 162.76 89.62) (width 0.5) (layer "B.Cu") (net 16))
 (segment (start 164.65 76.31) (end 164.65 78.15) (width 0.5) (layer "F.Cu") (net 12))
 (segment (start 176.12 89.62) (end 178 89.62) (width 0.5) (layer "F.Cu") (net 12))
 (segment (start 164.65 78.15) (end 176.12 89.62) (width 0.5) (layer "F.Cu") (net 12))
 (segment (start 167.19 77.69) (end 174.04 84.54) (width 0.5) (layer "F.Cu") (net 11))
 (segment (start 167.19 76.31) (end 167.19 77.69) (width 0.5) (layer "F.Cu") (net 11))
 (segment (start 174.04 84.54) (end 178 84.54) (width 0.5) (layer "F.Cu") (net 11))
 (segment (start 174.81 76.31) (end 174.81 80.11) (width 0.5) (layer "B.Cu") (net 17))
 (segment (start 174.81 80.11) (end 162.76 92.16) (width 0.5) (layer "B.Cu") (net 17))
 (segment (start 186.5 64.88) (end 186.5 49.985) (width 0.5) (layer "F.Cu") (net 18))
 (segment (start 186.5 49.985) (end 184.885 48.37) (width 0.5) (layer "F.Cu") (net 18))
 (segment (start 150 53.795) (end 150 54.175) (width 0.5) (layer "B.Cu") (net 41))
 (segment (start 155.425 48.37) (end 150 53.795) (width 0.5) (layer "B.Cu") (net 41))
 (segment (start 150 54.175) (end 155.025 59.2) (width 0.5) (layer "B.Cu") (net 41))
 (segment (start 142 54) (end 139.81 56.19) (width 0.5) (layer "F.Cu") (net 3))
 (segment (start 160.505 49.495) (end 156 54) (width 0.5) (layer "F.Cu") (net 3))
 (segment (start 156 54) (end 142 54) (width 0.5) (layer "F.Cu") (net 3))
 (segment (start 160.505 48.37) (end 160.505 49.495) (width 0.5) (layer "F.Cu") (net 3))
 (segment (start 139.81 56.19) (end 138.5 56.19) (width 0.5) (layer "F.Cu") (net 3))
 (segment (start 157.965 50.11875) (end 155.08375 53) (width 0.5) (layer "F.Cu") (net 39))
 (segment (start 157.965 48.37) (end 157.965 50.11875) (width 0.5) (layer "F.Cu") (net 39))
 (segment (start 155.08375 53) (end 139.5 53) (width 0.5) (layer "F.Cu") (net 39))
 (segment (start 139.5 53) (end 136.5 56) (width 0.5) (layer "F.Cu") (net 39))
 (segment (start 136.5 56) (end 135 56) (width 0.5) (layer "F.Cu") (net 39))
 (segment (start 186.5 82.66) (end 186.5 95.015) (width 0.5) (layer "F.Cu") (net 25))
 (segment (start 186.5 95.015) (end 184.885 96.63) (width 0.5) (layer "F.Cu") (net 25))
 (segment (start 167.105 54.105) (end 167.19 54.19) (width 0.5) (layer "F.Cu") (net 37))
 (segment (start 167.105 48.37) (end 167.105 54.105) (width 0.5) (layer "F.Cu") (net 37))
 (segment (start 185 83.898) (end 185 93.975) (width 0.5) (layer "F.Cu") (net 24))
 (segment (start 185.199 83.699) (end 185 83.898) (width 0.5) (layer "F.Cu") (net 24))
 (segment (start 186.5 80.12) (end 185.199 81.421) (width 0.5) (layer "F.Cu") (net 24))
 (segment (start 185.199 81.421) (end 185.199 83.699) (width 0.5) (layer "F.Cu") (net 24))
 (segment (start 185 93.975) (end 182.345 96.63) (width 0.5) (layer "F.Cu") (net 24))
 (segment (start 174.81 50.995) (end 172.185 48.37) (width 0.5) (layer "F.Cu") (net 35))
 (segment (start 174.81 54.19) (end 174.81 50.995) (width 0.5) (layer "F.Cu") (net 35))
 (segment (start 185 51) (end 184.975 51) (width 0.5) (layer "F.Cu") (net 19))
 (segment (start 186.5 67.42) (end 185 65.92) (width 0.5) (layer "F.Cu") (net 19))
 (segment (start 185 65.92) (end 185 51) (width 0.5) (layer "F.Cu") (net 19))
 (segment (start 184.975 51) (end 182.345 48.37) (width 0.5) (layer "F.Cu") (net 19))
 (segment (start 184 80.08) (end 184 92.435) (width 0.5) (layer "F.Cu") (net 23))
 (segment (start 184 92.435) (end 179.805 96.63) (width 0.5) (layer "F.Cu") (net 23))
 (segment (start 186.5 77.58) (end 184 80.08) (width 0.5) (layer "F.Cu") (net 23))
 (segment (start 172.27 54.19) (end 172.27 50.995) (width 0.5) (layer "F.Cu") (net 36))
 (segment (start 172.27 50.995) (end 169.645 48.37) (width 0.5) (layer "F.Cu") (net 36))
 (segment (start 127 72.96) (end 124.04 72.96) (width 0.5) (layer "F.Cu") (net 5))
 (segment (start 146.38 83.525) (end 144.975 83.525) (width 0.5) (layer "F.Cu") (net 5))
 (segment (start 123.5 84) (end 123.975 83.525) (width 0.5) (layer "F.Cu") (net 5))
 (segment (start 123.5 73.5) (end 123.5 84) (width 0.5) (layer "F.Cu") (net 5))
 (segment (start 124.04 72.96) (end 123.5 73.5) (width 0.5) (layer "F.Cu") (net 5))
 (segment (start 123.975 83.525) (end 144.975 83.525) (width 0.5) (layer "F.Cu") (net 5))
 (segment (start 159.485 96.63) (end 146.38 83.525) (width 0.5) (layer "F.Cu") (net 5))
 (segment (start 158.5 74.5) (end 149.475 83.525) (width 0.5) (layer "B.Cu") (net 5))
 (segment (start 162.11 54.19) (end 162.11 56.39) (width 0.5) (layer "B.Cu") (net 5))
 (segment (start 158.5 60) (end 158.5 74.5) (width 0.5) (layer "B.Cu") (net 5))
 (segment (start 162.11 56.39) (end 158.5 60) (width 0.5) (layer "B.Cu") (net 5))
 (segment (start 149.475 83.525) (end 144.975 83.525) (width 0.5) (layer "B.Cu") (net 5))
 (segment (start 183 69) (end 183 53.5) (width 0.5) (layer "F.Cu") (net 21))
 (segment (start 186.5 72.5) (end 183 69) (width 0.5) (layer "F.Cu") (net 21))
 (segment (start 180 50.5) (end 176.855 50.5) (width 0.5) (layer "F.Cu") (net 21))
 (segment (start 176.855 50.5) (end 174.725 48.37) (width 0.5) (layer "F.Cu") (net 21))
 (segment (start 183 53.5) (end 180 50.5) (width 0.5) (layer "F.Cu") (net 21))
 (segment (start 148.5 52.755) (end 148.5 71.5) (width 0.5) (layer "B.Cu") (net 8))
 (segment (start 152.885 48.37) (end 148.5 52.755) (width 0.5) (layer "B.Cu") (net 8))
 (segment (start 148.5 71.5) (end 144.5 75.5) (width 0.5) (layer "B.Cu") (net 8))
 (segment (start 144.5 75.5) (end 127 75.5) (width 0.5) (layer "B.Cu") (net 8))
 (segment (start 178.516 49.621) (end 177.265 48.37) (width 0.5) (layer "F.Cu") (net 20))
 (segment (start 180.879 49.621) (end 178.516 49.621) (width 0.5) (layer "F.Cu") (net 20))
 (segment (start 184 52.5) (end 181 49.5) (width 0.5) (layer "F.Cu") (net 20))
 (segment (start 186.5 69.96) (end 184 67.46) (width 0.5) (layer "F.Cu") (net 20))
 (segment (start 184 67.46) (end 184 52.5) (width 0.5) (layer "F.Cu") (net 20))
 (segment (start 181 49.5) (end 180.879 49.621) (width 0.5) (layer "F.Cu") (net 20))
 (segment (start 132.5 66) (end 128 70.5) (width 0.5) (layer "B.Cu") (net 9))
 (segment (start 122 78) (end 122.04 78.04) (width 0.5) (layer "B.Cu") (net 9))
 (segment (start 128 70.5) (end 122.5 70.5) (width 0.5) (layer "B.Cu") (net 9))
 (segment (start 122.04 78.04) (end 127 78.04) (width 0.5) (layer "B.Cu") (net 9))
 (segment (start 122.5 70.5) (end 122 71) (width 0.5) (layer "B.Cu") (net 9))
 (segment (start 122 71) (end 122 78) (width 0.5) (layer "B.Cu") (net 9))
 (segment (start 150.345 48.37) (end 147.715 51) (width 0.5) (layer "B.Cu") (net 9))
 (segment (start 147.715 51) (end 132.5 51) (width 0.5) (layer "B.Cu") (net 9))
 (segment (start 132.5 51) (end 132.5 66) (width 0.5) (layer "B.Cu") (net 9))
 (segment (start 158.209636 94.701) (end 158.008636 94.5) (width 0.5) (layer "B.Cu") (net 7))
 (segment (start 158 94.5) (end 150 86.5) (width 0.5) (layer "B.Cu") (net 7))
 (segment (start 170.256 94.701) (end 158.209636 94.701) (width 0.5) (layer "B.Cu") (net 7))
 (segment (start 158.008636 94.5) (end 158 94.5) (width 0.5) (layer "B.Cu") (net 7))
 (segment (start 142.5 86.5) (end 142.5 78.5) (width 0.5) (layer "B.Cu") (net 7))
 (segment (start 150 86.5) (end 142.5 86.5) (width 0.5) (layer "B.Cu") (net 7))
 (segment (start 172.185 96.63) (end 170.256 94.701) (width 0.5) (layer "B.Cu") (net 7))
 (segment (start 142.5 78.5) (end 144.92 78.5) (width 0.5) (layer "B.Cu") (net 7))
 (segment (start 144.92 78.5) (end 144.975 78.445) (width 0.5) (layer "B.Cu") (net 7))
 (segment (start 163.045 48.37) (end 155.415 56) (width 0.5) (layer "F.Cu") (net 1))
 (segment (start 155.415 56) (end 142 56) (width 0.5) (layer "F.Cu") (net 1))
 (segment (start 186.5 75.04) (end 182.5 79.04) (width 0.5) (layer "F.Cu") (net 22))
 (segment (start 182.5 91.395) (end 177.265 96.63) (width 0.5) (layer "F.Cu") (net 22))
 (segment (start 182.5 79.04) (end 182.5 91.395) (width 0.5) (layer "F.Cu") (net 22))
 (segment (start 135 63.62) (end 135 70.205) (width 0.5) (layer "F.Cu") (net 40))
 (segment (start 135 70.205) (end 134.68 70.525) (width 0.5) (layer "F.Cu") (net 40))
 (segment (start 138.5 63.81) (end 138.5 69.245) (width 0.5) (layer "F.Cu") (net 4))
 (segment (start 138.5 69.245) (end 137.22 70.525) (width 0.5) (layer "F.Cu") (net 4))
 (segment (start 142 63.62) (end 142 70.225) (width 0.5) (layer "F.Cu") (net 2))
 (segment (start 142 70.225) (end 142.3 70.525) (width 0.5) (layer "F.Cu") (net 2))
 (segment (start 172.27 61.81) (end 172.27 68.69) (width 0.5) (layer "F.Cu") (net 30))
 (segment (start 164.65 61.81) (end 164.65 68.69) (width 0.5) (layer "F.Cu") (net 27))
 (segment (start 177.35 61.81) (end 177.35 68.69) (width 0.5) (layer "F.Cu") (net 32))
 (segment (start 169.73 61.81) (end 169.73 68.69) (width 0.5) (layer "F.Cu") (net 29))
 (segment (start 162.11 61.81) (end 162.11 68.69) (width 0.5) (layer "F.Cu") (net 26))
 (segment (start 167.19 61.81) (end 167.19 68.69) (width 0.5) (layer "F.Cu") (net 28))
 (segment (start 174.81 61.81) (end 174.81 68.69) (width 0.5) (layer "F.Cu") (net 31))
 (segment (start 164.65 54.19) (end 171.019 60.559) (width 0.5) (layer "B.Cu") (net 38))
 (segment (start 173.559 61.329818) (end 173.559 62.359) (width 0.5) (layer "B.Cu") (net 38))
 (segment (start 172.788182 60.559) (end 173.559 61.329818) (width 0.5) (layer "B.Cu") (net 38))
 (segment (start 173.559 62.359) (end 179.89 68.69) (width 0.5) (layer "B.Cu") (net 38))
 (segment (start 171.019 60.559) (end 172.788182 60.559) (width 0.5) (layer "B.Cu") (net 38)))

